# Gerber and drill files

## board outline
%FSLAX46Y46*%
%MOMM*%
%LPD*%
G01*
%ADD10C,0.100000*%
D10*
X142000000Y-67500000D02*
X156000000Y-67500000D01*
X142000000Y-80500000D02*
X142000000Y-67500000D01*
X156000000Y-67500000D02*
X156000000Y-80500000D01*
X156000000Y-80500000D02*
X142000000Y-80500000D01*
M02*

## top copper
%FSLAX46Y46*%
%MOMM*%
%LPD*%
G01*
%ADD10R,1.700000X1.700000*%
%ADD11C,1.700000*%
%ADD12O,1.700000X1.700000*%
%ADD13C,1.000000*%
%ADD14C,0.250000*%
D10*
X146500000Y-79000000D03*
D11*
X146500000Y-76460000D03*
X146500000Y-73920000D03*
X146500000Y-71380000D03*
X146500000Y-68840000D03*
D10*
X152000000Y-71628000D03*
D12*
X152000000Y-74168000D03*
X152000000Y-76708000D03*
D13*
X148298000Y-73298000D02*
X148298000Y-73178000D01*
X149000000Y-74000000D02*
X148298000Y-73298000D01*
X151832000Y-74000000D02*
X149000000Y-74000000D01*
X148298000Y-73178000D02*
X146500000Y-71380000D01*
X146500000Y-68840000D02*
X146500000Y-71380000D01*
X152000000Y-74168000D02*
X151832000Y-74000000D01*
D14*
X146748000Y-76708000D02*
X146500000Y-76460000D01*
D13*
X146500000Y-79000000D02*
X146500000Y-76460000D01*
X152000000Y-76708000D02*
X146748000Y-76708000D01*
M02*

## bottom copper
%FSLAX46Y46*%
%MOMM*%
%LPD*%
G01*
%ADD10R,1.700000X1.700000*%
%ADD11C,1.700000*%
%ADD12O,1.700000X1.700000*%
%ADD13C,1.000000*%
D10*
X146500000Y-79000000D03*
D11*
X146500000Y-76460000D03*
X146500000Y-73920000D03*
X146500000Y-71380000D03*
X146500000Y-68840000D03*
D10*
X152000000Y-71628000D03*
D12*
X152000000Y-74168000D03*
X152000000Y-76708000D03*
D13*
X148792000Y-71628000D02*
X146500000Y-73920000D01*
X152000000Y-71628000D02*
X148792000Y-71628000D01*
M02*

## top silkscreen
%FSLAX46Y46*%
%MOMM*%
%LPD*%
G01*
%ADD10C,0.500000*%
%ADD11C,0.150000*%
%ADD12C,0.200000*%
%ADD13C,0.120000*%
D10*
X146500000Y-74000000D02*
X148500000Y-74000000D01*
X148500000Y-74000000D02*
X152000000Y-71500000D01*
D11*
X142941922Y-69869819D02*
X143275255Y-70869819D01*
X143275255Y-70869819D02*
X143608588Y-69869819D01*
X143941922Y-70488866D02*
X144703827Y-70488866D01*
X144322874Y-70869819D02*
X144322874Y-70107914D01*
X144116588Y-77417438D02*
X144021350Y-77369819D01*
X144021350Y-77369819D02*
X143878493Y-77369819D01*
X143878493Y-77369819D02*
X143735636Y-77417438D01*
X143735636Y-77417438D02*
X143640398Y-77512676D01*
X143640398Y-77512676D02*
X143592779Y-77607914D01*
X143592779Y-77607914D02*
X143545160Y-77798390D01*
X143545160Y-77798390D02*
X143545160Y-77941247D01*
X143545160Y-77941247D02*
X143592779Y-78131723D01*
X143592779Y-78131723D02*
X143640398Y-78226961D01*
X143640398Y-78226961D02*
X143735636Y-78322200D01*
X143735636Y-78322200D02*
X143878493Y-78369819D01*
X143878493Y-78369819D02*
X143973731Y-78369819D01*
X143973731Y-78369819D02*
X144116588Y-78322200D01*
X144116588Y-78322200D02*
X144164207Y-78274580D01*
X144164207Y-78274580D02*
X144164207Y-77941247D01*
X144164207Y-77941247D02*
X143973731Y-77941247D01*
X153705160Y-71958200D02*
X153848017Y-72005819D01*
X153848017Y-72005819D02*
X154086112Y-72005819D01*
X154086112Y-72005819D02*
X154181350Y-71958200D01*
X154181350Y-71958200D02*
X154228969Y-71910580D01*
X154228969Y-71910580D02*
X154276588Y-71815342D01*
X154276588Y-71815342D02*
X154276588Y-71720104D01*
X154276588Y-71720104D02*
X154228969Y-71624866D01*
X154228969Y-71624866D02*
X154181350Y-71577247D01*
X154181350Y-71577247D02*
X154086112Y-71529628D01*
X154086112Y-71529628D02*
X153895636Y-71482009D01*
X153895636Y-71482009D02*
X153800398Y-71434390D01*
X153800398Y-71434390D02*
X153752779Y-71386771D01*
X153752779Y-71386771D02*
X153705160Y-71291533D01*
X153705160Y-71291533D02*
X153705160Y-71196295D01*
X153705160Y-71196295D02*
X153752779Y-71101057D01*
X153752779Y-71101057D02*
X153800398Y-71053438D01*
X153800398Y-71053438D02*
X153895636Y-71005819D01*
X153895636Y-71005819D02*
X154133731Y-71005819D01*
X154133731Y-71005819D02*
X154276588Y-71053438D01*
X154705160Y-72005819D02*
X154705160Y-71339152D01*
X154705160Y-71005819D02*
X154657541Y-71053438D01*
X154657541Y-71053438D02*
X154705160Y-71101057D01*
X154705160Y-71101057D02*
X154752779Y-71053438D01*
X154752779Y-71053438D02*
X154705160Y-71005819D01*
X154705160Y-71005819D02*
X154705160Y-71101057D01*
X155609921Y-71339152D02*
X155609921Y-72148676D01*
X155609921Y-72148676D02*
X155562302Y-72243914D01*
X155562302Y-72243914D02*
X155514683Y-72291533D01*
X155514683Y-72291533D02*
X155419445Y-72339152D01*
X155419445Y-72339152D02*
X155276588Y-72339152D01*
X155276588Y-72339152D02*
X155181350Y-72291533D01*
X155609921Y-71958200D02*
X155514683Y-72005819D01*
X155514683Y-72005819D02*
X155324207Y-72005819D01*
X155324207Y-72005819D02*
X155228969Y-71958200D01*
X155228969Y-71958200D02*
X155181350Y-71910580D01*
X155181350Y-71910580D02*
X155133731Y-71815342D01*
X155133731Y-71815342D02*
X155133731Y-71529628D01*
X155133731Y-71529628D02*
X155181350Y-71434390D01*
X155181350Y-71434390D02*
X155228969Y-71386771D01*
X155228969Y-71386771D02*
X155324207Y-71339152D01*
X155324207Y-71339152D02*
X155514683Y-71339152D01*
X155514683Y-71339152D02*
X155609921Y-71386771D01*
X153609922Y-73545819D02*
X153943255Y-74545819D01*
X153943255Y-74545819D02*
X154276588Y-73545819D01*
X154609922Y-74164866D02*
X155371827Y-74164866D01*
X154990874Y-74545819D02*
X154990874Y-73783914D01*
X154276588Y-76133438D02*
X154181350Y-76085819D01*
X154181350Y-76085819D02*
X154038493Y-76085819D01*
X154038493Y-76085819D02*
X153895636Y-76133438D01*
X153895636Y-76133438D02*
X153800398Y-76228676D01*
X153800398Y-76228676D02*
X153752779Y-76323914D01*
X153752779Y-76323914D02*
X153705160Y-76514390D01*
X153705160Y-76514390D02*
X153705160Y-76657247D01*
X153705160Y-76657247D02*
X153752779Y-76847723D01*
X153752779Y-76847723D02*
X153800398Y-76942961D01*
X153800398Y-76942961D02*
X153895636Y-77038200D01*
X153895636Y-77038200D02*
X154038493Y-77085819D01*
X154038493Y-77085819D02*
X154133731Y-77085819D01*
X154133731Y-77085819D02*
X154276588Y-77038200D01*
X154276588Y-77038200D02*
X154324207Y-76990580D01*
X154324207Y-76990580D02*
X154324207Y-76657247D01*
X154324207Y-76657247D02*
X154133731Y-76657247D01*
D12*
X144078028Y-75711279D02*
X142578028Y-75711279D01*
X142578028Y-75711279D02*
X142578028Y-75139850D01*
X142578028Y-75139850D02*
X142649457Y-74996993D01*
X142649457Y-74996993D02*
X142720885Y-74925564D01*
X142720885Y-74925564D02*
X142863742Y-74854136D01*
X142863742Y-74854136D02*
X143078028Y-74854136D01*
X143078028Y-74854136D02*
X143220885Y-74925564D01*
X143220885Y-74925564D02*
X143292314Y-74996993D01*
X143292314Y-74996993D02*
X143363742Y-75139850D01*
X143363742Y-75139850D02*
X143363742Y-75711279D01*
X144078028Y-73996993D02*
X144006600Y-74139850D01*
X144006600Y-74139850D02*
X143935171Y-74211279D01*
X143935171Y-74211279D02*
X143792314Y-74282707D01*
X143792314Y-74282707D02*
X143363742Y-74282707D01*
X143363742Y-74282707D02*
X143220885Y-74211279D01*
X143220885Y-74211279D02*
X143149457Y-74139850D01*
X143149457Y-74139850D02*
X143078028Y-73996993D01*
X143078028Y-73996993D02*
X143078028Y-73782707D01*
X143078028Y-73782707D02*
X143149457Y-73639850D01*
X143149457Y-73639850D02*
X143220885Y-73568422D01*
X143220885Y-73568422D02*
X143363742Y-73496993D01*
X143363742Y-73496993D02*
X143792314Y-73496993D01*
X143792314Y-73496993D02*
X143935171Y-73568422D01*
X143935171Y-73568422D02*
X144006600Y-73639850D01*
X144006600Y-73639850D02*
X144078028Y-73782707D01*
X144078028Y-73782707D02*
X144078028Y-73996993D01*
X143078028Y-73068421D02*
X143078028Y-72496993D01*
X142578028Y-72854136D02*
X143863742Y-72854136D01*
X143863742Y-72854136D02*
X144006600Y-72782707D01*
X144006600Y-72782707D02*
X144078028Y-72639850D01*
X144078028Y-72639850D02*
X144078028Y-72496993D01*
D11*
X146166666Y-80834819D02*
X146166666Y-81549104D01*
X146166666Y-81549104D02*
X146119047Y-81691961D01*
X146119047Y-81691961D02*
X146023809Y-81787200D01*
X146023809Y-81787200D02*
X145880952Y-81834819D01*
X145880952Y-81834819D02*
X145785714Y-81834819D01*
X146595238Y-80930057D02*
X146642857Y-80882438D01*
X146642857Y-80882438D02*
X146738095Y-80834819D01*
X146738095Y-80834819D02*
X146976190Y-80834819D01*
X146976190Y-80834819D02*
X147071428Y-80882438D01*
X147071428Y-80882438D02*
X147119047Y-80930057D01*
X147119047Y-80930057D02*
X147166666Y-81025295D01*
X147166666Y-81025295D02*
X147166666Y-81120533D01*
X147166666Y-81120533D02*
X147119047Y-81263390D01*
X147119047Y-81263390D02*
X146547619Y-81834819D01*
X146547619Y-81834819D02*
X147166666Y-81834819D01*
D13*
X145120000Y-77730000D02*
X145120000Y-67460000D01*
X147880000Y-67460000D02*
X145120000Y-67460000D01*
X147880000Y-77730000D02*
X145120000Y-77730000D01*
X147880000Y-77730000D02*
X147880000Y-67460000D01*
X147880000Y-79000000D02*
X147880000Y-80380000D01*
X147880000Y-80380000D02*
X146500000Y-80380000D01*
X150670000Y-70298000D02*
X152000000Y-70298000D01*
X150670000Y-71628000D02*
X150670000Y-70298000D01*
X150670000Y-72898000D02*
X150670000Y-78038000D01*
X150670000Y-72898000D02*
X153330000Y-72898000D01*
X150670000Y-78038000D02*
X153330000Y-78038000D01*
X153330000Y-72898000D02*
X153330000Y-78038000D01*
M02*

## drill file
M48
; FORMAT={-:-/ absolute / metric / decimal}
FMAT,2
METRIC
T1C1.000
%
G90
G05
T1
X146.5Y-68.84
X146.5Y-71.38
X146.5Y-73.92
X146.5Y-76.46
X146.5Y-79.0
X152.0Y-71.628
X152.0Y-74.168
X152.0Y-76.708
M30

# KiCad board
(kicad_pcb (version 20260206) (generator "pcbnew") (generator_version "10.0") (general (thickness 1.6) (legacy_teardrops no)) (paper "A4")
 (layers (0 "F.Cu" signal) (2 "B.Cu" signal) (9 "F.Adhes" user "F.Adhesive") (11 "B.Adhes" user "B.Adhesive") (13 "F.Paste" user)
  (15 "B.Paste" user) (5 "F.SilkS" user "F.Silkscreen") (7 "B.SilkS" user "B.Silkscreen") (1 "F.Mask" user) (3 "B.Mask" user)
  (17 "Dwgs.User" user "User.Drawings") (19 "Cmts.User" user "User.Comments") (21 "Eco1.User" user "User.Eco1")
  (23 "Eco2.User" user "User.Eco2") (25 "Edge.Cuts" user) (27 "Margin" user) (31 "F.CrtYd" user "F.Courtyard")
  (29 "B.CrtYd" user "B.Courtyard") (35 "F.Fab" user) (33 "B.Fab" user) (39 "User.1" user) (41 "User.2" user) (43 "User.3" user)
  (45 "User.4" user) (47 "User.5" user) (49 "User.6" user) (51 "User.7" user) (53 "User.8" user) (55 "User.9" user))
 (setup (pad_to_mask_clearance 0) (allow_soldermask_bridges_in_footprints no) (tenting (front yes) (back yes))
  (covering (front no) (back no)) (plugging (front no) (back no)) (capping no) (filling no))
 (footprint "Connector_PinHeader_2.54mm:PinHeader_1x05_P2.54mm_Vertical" (layer "F.Cu") (at 146.5 79 180)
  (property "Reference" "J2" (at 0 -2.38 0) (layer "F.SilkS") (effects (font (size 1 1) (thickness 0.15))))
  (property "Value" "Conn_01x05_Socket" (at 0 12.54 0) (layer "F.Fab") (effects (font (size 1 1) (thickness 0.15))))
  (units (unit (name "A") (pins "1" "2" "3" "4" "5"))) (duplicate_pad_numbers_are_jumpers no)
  (fp_line (start 1.38 1.27) (end 1.38 11.54) (stroke (width 0.12) (type solid)) (layer "F.SilkS"))
  (fp_line (start -1.38 11.54) (end 1.38 11.54) (stroke (width 0.12) (type solid)) (layer "F.SilkS"))
  (fp_line (start -1.38 1.27) (end 1.38 1.27) (stroke (width 0.12) (type solid)) (layer "F.SilkS"))
  (fp_line (start -1.38 1.27) (end -1.38 11.54) (stroke (width 0.12) (type solid)) (layer "F.SilkS"))
  (fp_line (start -1.38 0) (end -1.38 -1.38) (stroke (width 0.12) (type solid)) (layer "F.SilkS"))
  (fp_line (start -1.38 -1.38) (end 0 -1.38) (stroke (width 0.12) (type solid)) (layer "F.SilkS"))
  (pad "1" thru_hole rect (at 0 0 180) (size 1.7 1.7) (drill 1) (layers "*.Cu" "*.Mask") (remove_unused_layers no) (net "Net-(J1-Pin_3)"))
  (pad "2" thru_hole circle (at 0 2.54 180) (size 1.7 1.7) (drill 1) (layers "*.Cu" "*.Mask") (remove_unused_layers no)
   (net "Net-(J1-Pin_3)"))
  (pad "3" thru_hole circle (at 0 5.08 180) (size 1.7 1.7) (drill 1) (layers "*.Cu" "*.Mask") (remove_unused_layers no)
   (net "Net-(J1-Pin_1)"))
  (pad "4" thru_hole circle (at 0 7.62 180) (size 1.7 1.7) (drill 1) (layers "*.Cu" "*.Mask") (remove_unused_layers no)
   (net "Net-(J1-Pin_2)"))
  (pad "5" thru_hole circle (at 0 10.16 180) (size 1.7 1.7) (drill 1) (layers "*.Cu" "*.Mask") (remove_unused_layers no)
   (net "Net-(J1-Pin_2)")))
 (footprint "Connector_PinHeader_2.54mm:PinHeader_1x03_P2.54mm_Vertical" (layer "F.Cu") (at 152 71.628)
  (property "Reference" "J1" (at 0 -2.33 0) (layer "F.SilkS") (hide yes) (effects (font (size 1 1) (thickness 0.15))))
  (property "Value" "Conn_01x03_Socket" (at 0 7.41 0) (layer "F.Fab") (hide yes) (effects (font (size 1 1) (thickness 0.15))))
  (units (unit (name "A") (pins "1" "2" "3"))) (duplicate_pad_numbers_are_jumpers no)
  (fp_line (start -1.33 -1.33) (end 0 -1.33) (stroke (width 0.12) (type solid)) (layer "F.SilkS"))
  (fp_line (start -1.33 0) (end -1.33 -1.33) (stroke (width 0.12) (type solid)) (layer "F.SilkS"))
  (fp_line (start -1.33 1.27) (end -1.33 6.41) (stroke (width 0.12) (type solid)) (layer "F.SilkS"))
  (fp_line (start -1.33 1.27) (end 1.33 1.27) (stroke (width 0.12) (type solid)) (layer "F.SilkS"))
  (fp_line (start -1.33 6.41) (end 1.33 6.41) (stroke (width 0.12) (type solid)) (layer "F.SilkS"))
  (fp_line (start 1.33 1.27) (end 1.33 6.41) (stroke (width 0.12) (type solid)) (layer "F.SilkS"))
  (pad "1" thru_hole rect (at 0 0) (size 1.7 1.7) (drill 1) (layers "*.Cu" "*.Mask") (remove_unused_layers no) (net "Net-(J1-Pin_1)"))
  (pad "2" thru_hole oval (at 0 2.54) (size 1.7 1.7) (drill 1) (layers "*.Cu" "*.Mask") (remove_unused_layers no) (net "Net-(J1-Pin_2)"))
  (pad "3" thru_hole oval (at 0 5.08) (size 1.7 1.7) (drill 1) (layers "*.Cu" "*.Mask") (remove_unused_layers no) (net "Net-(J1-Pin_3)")))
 (gr_line (start 146.5 74) (end 148.5 74) (stroke (width 0.5) (type solid)) (layer "F.SilkS"))
 (gr_line (start 148.5 74) (end 152 71.5) (stroke (width 0.5) (type solid)) (layer "F.SilkS"))
 (gr_line (start 142 67.5) (end 156 67.5) (stroke (width 0.1) (type solid)) (layer "Edge.Cuts"))
 (gr_line (start 142 80.5) (end 142 67.5) (stroke (width 0.1) (type solid)) (layer "Edge.Cuts"))
 (gr_line (start 156 67.5) (end 156 80.5) (stroke (width 0.1) (type solid)) (layer "Edge.Cuts"))
 (gr_line (start 156 80.5) (end 142 80.5) (stroke (width 0.1) (type solid)) (layer "Edge.Cuts"))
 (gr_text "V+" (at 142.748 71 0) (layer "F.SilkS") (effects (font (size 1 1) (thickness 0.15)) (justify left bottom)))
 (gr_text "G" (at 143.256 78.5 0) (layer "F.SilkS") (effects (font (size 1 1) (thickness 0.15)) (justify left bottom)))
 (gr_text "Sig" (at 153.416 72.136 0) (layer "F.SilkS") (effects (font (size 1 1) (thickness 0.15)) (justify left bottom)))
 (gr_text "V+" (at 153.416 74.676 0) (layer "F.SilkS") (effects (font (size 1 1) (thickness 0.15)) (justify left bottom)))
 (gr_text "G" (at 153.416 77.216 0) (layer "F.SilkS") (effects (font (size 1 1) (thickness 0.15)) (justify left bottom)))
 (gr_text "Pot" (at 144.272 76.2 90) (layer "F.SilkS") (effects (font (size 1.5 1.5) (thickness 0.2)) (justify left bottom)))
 (segment (start 148.792 71.628) (end 146.5 73.92) (width 1) (layer "B.Cu") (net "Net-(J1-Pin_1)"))
 (segment (start 152 71.628) (end 148.792 71.628) (width 1) (layer "B.Cu") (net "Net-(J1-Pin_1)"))
 (segment (start 148.298 73.298) (end 148.298 73.178) (width 1) (layer "F.Cu") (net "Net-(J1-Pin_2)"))
 (segment (start 149 74) (end 148.298 73.298) (width 1) (layer "F.Cu") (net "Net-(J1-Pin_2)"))
 (segment (start 151.832 74) (end 149 74) (width 1) (layer "F.Cu") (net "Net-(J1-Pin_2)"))
 (segment (start 148.298 73.178) (end 146.5 71.38) (width 1) (layer "F.Cu") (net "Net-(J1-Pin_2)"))
 (segment (start 146.5 68.84) (end 146.5 71.38) (width 1) (layer "F.Cu") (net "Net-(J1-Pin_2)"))
 (segment (start 152 74.168) (end 151.832 74) (width 1) (layer "F.Cu") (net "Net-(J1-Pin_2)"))
 (segment (start 146.748 76.708) (end 146.5 76.46) (width 0.25) (layer "F.Cu") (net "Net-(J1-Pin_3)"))
 (segment (start 146.5 79) (end 146.5 76.46) (width 1) (layer "F.Cu") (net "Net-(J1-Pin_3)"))
 (segment (start 152 76.708) (end 146.748 76.708) (width 1) (layer "F.Cu") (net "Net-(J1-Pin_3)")))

